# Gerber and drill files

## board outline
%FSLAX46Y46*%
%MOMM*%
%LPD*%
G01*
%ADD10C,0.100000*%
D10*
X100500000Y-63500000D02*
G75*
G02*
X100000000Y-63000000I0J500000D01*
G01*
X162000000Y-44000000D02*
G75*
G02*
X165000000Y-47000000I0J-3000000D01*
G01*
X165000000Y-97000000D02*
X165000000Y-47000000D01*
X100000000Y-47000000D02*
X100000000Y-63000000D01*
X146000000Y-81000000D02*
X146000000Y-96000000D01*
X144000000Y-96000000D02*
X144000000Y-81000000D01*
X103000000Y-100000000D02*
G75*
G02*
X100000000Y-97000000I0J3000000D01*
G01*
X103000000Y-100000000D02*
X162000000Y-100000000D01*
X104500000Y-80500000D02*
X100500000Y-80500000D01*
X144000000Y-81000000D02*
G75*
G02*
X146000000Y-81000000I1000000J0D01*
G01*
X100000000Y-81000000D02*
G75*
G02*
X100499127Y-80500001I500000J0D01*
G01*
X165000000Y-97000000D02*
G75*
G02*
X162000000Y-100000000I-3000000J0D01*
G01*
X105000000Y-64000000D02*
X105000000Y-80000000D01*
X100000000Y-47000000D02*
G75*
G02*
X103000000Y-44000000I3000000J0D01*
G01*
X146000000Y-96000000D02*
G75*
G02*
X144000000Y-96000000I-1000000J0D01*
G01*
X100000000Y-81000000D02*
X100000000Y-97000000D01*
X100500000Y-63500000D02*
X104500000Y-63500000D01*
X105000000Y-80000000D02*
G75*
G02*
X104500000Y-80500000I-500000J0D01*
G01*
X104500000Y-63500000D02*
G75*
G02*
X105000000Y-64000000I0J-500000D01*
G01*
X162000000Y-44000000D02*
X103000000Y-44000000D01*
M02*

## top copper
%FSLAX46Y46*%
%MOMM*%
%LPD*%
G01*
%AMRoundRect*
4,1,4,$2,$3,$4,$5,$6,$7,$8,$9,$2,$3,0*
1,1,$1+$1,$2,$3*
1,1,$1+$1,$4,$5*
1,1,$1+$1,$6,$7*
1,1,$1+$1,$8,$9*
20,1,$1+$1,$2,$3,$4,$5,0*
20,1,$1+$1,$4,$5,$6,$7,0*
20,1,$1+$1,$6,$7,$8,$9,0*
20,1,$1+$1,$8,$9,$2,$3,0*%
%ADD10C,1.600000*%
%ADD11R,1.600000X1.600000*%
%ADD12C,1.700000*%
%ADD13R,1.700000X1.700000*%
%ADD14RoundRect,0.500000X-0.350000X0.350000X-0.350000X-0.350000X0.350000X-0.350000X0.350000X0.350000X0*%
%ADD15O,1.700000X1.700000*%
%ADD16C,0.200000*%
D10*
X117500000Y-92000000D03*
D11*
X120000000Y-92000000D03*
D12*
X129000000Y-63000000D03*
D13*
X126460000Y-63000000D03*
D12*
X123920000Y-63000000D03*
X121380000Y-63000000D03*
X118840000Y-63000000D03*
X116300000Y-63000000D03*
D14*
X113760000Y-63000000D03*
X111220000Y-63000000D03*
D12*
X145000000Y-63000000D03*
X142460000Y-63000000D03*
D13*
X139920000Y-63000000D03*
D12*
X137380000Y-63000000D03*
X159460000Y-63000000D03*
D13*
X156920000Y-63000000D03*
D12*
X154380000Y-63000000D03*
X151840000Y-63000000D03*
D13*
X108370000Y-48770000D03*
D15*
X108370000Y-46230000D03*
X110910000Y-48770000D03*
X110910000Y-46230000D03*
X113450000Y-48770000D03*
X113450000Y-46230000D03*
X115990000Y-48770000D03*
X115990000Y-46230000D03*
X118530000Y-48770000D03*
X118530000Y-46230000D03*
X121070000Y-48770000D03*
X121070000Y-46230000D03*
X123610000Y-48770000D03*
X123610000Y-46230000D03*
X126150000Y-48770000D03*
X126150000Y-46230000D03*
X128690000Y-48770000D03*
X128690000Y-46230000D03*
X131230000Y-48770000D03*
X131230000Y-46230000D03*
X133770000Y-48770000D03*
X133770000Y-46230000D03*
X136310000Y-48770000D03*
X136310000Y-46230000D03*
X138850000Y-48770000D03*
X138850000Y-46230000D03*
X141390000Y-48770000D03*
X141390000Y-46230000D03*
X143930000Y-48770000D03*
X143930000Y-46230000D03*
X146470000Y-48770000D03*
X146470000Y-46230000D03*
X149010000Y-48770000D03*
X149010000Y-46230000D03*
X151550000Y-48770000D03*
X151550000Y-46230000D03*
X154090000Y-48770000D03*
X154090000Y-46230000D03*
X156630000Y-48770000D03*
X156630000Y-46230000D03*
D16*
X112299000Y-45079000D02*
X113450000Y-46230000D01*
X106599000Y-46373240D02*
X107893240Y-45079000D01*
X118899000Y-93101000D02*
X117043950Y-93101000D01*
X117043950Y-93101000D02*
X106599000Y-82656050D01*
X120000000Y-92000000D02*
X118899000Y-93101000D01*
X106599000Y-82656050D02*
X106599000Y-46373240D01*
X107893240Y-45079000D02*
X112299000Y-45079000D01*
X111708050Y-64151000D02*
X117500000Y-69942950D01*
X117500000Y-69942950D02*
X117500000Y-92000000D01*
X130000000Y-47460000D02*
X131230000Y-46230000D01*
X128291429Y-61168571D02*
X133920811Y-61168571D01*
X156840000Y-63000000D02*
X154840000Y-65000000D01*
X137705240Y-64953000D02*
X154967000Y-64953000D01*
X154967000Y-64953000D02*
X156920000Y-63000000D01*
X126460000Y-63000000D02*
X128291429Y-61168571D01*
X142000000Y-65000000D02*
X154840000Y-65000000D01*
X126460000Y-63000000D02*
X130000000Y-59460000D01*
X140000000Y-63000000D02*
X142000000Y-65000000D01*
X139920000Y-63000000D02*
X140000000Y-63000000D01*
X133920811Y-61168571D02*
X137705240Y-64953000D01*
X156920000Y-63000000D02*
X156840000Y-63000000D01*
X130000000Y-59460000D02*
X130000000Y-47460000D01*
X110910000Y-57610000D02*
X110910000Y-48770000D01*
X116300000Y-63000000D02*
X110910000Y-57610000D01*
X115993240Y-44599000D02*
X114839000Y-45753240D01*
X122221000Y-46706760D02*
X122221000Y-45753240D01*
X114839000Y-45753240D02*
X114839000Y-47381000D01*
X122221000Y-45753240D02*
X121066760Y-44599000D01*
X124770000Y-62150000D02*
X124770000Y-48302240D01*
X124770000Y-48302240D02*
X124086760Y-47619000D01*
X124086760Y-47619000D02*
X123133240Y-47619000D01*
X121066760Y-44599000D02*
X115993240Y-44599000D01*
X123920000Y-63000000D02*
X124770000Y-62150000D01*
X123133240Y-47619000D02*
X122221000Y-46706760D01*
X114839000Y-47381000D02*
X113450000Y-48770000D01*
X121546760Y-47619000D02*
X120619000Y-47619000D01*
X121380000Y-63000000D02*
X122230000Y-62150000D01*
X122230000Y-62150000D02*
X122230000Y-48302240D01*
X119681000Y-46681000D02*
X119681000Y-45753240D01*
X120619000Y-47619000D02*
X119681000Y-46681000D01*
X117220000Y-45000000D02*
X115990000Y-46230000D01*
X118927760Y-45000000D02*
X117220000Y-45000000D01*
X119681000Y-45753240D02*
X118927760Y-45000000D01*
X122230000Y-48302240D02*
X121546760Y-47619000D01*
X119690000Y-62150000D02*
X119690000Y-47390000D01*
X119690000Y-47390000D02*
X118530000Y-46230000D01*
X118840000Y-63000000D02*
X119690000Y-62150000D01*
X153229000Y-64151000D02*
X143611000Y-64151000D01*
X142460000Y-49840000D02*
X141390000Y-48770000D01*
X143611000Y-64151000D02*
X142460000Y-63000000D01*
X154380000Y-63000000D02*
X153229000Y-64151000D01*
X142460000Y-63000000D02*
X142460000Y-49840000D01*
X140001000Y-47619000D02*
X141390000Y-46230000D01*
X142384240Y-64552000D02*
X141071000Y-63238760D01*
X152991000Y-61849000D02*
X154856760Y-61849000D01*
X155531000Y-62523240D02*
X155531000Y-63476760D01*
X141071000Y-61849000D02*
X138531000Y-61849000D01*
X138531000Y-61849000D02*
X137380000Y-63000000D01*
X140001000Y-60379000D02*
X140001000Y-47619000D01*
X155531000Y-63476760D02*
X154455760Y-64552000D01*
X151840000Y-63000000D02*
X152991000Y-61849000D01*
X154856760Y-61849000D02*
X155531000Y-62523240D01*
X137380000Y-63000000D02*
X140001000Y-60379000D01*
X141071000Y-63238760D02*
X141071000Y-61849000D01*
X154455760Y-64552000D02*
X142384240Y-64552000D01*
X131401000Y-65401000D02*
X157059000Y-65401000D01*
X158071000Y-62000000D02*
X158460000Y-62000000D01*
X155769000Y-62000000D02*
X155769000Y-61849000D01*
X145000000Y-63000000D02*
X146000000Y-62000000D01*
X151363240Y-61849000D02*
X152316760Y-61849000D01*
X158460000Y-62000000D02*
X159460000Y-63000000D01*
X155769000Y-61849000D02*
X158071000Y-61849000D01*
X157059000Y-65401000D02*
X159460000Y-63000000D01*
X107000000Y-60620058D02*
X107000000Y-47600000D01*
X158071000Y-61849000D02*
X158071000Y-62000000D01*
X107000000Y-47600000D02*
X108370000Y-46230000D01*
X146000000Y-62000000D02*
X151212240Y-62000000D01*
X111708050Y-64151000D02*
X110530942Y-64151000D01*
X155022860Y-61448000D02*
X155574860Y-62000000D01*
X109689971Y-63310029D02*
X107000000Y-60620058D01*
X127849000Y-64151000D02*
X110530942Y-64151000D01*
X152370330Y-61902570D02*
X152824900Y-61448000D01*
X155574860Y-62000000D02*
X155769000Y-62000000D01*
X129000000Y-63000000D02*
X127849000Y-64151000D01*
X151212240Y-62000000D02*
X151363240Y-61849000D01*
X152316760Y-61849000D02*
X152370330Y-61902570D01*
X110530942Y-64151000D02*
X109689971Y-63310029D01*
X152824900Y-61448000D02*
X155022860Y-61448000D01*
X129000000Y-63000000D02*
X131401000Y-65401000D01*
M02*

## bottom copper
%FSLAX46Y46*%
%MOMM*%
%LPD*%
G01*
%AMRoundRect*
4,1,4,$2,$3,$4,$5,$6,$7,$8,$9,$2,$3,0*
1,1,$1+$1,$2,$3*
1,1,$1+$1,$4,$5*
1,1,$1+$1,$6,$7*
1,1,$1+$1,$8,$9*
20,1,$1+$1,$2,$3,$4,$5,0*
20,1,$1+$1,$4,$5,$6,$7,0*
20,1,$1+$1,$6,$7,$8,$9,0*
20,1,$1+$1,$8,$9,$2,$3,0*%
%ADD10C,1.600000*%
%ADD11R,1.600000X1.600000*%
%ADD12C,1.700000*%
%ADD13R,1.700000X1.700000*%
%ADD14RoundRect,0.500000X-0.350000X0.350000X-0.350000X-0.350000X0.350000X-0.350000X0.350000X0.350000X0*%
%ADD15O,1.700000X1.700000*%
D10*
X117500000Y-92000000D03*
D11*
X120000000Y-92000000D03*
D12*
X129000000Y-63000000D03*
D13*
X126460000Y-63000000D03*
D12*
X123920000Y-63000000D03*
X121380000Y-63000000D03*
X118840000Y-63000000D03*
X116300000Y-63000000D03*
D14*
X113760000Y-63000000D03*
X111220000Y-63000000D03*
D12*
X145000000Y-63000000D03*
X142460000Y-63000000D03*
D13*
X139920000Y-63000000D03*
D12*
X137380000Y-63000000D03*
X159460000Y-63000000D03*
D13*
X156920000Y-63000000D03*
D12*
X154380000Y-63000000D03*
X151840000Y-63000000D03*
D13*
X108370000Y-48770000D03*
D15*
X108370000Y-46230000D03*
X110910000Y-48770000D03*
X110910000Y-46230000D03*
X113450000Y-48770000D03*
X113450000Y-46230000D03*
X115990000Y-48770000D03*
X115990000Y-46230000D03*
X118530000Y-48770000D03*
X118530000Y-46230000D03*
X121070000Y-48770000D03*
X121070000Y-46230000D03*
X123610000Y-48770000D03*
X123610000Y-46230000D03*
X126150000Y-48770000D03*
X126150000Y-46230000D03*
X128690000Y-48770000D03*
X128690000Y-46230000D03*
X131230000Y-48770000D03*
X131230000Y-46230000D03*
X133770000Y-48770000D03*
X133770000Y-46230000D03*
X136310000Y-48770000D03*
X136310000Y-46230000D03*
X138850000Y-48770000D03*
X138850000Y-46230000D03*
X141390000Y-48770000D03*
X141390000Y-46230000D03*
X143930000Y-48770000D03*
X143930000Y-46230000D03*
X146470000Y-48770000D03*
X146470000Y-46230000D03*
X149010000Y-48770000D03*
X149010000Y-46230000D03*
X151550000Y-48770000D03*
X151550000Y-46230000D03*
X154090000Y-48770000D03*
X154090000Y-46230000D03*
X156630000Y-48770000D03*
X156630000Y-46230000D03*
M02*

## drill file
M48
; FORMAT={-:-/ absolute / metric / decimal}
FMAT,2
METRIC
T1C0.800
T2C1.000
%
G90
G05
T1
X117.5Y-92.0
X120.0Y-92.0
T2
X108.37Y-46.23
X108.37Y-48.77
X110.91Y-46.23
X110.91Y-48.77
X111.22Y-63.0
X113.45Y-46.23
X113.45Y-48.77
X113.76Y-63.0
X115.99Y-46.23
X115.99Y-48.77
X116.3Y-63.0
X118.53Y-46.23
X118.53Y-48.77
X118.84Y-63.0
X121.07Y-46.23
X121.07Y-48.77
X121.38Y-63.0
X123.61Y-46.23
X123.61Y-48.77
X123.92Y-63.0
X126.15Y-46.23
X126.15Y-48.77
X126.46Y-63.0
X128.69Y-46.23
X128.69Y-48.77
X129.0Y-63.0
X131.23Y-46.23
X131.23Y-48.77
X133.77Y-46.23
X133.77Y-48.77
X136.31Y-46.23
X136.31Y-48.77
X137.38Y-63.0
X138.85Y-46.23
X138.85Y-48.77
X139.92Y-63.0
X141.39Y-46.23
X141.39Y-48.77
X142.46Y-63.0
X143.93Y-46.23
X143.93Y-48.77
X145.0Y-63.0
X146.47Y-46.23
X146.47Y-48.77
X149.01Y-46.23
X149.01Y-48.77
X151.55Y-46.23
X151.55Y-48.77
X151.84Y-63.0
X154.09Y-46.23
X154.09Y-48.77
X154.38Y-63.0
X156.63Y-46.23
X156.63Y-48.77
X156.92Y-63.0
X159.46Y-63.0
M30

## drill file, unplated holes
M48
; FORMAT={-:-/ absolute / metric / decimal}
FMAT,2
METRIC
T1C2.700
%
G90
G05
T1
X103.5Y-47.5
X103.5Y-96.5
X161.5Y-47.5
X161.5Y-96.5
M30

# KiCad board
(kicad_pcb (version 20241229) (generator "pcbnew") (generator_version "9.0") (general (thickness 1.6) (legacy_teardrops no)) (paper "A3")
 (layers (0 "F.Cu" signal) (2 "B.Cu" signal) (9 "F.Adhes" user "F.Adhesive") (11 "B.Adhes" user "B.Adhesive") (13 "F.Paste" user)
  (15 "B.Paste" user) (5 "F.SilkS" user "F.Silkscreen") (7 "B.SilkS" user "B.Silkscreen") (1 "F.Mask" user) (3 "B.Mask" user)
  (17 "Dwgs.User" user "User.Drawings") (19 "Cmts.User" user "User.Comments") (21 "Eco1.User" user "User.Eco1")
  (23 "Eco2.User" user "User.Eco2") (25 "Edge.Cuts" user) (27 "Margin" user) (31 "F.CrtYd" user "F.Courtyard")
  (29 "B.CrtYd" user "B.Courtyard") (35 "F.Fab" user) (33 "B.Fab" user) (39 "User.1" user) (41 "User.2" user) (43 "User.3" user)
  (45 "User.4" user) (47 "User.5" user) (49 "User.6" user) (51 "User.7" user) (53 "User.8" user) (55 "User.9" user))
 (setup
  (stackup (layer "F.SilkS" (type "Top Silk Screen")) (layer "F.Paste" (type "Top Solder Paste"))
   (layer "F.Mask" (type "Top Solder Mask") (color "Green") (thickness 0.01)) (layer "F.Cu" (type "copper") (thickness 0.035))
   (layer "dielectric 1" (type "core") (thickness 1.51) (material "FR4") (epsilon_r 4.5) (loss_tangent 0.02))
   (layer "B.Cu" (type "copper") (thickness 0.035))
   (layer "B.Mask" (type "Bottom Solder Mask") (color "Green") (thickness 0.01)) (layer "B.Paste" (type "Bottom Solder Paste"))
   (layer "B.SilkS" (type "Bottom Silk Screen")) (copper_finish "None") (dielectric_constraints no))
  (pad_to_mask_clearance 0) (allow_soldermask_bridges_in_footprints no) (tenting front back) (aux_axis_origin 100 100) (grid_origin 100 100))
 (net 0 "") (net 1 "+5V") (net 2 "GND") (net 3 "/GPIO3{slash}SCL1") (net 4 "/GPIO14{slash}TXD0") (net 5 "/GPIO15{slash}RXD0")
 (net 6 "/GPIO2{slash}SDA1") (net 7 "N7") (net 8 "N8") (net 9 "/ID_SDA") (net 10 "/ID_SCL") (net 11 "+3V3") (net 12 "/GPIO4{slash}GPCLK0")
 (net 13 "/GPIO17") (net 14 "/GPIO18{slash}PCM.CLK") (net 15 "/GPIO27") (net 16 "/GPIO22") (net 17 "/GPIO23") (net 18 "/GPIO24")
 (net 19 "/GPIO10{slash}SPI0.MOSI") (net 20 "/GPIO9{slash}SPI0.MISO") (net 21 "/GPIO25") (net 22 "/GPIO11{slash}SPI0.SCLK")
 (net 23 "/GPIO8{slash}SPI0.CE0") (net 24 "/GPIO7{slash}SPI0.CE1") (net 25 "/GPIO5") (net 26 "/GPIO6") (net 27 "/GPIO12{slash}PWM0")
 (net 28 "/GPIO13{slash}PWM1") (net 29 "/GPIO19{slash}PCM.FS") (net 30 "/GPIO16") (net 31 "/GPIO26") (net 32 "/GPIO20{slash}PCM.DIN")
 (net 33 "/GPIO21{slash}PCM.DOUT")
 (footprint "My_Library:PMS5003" (layer "F.Cu") (at 121.38 63 -90)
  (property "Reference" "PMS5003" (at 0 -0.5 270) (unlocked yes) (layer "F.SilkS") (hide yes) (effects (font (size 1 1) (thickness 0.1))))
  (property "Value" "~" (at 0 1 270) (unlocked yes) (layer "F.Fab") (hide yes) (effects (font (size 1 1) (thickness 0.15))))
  (pad "1" thru_hole circle (at 0 -7.62 270) (size 1.7 1.7) (drill 1) (layers "*.Cu" "*.Mask") (remove_unused_layers no) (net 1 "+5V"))
  (pad "2" thru_hole rect (at 0 -5.08 270) (size 1.7 1.7) (drill 1) (layers "*.Cu" "*.Mask") (remove_unused_layers no) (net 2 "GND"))
  (pad "3" thru_hole circle (at 0 -2.54 270) (size 1.7 1.7) (drill 1) (layers "*.Cu" "*.Mask") (remove_unused_layers no)
   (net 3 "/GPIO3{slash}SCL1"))
  (pad "4" thru_hole circle (at 0 0 270) (size 1.7 1.7) (drill 1) (layers "*.Cu" "*.Mask") (remove_unused_layers no)
   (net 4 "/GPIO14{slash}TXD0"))
  (pad "5" thru_hole circle (at 0 2.54 270) (size 1.7 1.7) (drill 1) (layers "*.Cu" "*.Mask") (remove_unused_layers no)
   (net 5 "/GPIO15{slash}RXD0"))
  (pad "6" thru_hole circle (at 0 5.08 270) (size 1.7 1.7) (drill 1) (layers "*.Cu" "*.Mask") (remove_unused_layers no)
   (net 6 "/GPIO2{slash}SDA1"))
  (pad "7" thru_hole roundrect (at 0 7.62 270) (size 1.7 1.7) (drill 1) (layers "*.Cu" "*.Mask") (remove_unused_layers no)
   (roundrect_rratio 0.2941176471) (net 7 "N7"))
  (pad "8" thru_hole roundrect (at 0 10.16 270) (size 1.7 1.7) (drill 1) (layers "*.Cu" "*.Mask") (remove_unused_layers no)
   (roundrect_rratio 0.2941176471) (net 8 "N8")))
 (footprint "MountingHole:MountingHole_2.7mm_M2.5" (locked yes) (layer "F.Cu") (at 161.5 47.5)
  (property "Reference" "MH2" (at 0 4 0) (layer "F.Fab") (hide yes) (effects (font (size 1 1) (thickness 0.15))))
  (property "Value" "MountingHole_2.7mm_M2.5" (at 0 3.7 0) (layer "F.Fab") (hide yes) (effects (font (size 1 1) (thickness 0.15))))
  (pad "" np_thru_hole circle (at 0 0) (size 2.7 2.7) (drill 2.7) (layers "*.Cu" "*.Mask")))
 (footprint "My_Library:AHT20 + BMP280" (layer "F.Cu") (at 142.46 63 -90)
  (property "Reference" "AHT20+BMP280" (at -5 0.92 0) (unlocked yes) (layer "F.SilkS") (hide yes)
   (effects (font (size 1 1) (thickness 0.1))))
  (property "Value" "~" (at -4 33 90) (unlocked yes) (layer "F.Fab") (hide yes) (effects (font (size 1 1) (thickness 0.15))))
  (pad "1" thru_hole circle (at 0 -2.54 270) (size 1.7 1.7) (drill 1) (layers "*.Cu" "*.Mask") (remove_unused_layers no) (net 1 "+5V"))
  (pad "2" thru_hole circle (at 0 0 270) (size 1.7 1.7) (drill 1) (layers "*.Cu" "*.Mask") (remove_unused_layers no) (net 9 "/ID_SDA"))
  (pad "3" thru_hole rect (at 0 2.54 270) (size 1.7 1.7) (drill 1) (layers "*.Cu" "*.Mask") (remove_unused_layers no) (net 2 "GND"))
  (pad "4" thru_hole circle (at 0 5.08 270) (size 1.7 1.7) (drill 1) (layers "*.Cu" "*.Mask") (remove_unused_layers no) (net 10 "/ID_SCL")))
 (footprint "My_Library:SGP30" (layer "F.Cu") (at 156.92 63 -90)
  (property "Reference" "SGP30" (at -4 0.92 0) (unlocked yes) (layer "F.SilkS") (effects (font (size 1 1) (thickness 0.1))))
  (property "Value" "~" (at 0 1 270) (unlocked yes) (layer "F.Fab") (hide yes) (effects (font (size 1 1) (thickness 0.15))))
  (pad "1" thru_hole circle (at 0 -2.54 270) (size 1.7 1.7) (drill 1) (layers "*.Cu" "*.Mask") (remove_unused_layers no) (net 1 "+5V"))
  (pad "2" thru_hole rect (at 0 0 270) (size 1.7 1.7) (drill 1) (layers "*.Cu" "*.Mask") (remove_unused_layers no) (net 2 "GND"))
  (pad "3" thru_hole circle (at 0 2.54 270) (size 1.7 1.7) (drill 1) (layers "*.Cu" "*.Mask") (remove_unused_layers no) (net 9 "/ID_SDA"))
  (pad "4" thru_hole circle (at 0 5.08 270) (size 1.7 1.7) (drill 1) (layers "*.Cu" "*.Mask") (remove_unused_layers no) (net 10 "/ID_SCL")))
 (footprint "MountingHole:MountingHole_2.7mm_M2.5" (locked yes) (layer "F.Cu") (at 103.5 96.5)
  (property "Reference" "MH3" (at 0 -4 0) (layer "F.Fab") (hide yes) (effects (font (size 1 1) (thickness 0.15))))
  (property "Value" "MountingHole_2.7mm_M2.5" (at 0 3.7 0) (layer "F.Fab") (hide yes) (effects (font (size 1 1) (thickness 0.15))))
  (pad "" np_thru_hole circle (at 0 0) (size 2.7 2.7) (drill 2.7) (layers "*.Cu" "*.Mask")))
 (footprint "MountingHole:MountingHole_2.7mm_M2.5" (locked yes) (layer "F.Cu") (at 103.5 47.5)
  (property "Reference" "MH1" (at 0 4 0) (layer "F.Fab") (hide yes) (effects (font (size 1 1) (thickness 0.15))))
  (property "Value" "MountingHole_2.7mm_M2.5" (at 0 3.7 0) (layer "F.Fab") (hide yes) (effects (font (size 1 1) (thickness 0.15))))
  (pad "" np_thru_hole circle (at 0 0) (size 2.7 2.7) (drill 2.7) (layers "*.Cu" "*.Mask")))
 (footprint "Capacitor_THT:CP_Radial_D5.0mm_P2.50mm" (layer "F.Cu") (at 117.5 92)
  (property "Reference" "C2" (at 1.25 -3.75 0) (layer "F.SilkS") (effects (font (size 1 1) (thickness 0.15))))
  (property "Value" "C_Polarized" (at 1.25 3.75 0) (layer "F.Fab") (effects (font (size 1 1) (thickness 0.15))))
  (pad "1" thru_hole circle (at 0 0) (size 1.6 1.6) (drill 0.8) (layers "*.Cu" "*.Mask") (remove_unused_layers no) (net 1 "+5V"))
  (pad "2" thru_hole rect (at 2.5 0) (size 1.6 1.6) (drill 0.8) (layers "*.Cu" "*.Mask") (remove_unused_layers no) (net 2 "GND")))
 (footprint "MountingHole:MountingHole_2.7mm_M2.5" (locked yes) (layer "F.Cu") (at 161.5 96.5)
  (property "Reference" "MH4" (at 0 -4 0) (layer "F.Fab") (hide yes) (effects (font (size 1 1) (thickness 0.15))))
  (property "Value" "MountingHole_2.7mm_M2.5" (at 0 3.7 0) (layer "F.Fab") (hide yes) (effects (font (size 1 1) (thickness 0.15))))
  (pad "" np_thru_hole circle (at 0 0) (size 2.7 2.7) (drill 2.7) (layers "*.Cu" "*.Mask")))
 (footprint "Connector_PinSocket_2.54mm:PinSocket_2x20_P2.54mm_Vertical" (layer "B.Cu") (at 108.37 48.77 -90)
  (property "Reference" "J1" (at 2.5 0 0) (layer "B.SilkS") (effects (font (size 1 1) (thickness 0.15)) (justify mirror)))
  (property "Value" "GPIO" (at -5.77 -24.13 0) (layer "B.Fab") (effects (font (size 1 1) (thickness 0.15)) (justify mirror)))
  (pad "1" thru_hole rect (at 0 0 270) (size 1.7 1.7) (drill 1) (layers "*.Cu" "*.Mask") (remove_unused_layers no) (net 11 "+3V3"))
  (pad "2" thru_hole oval (at -2.54 0 270) (size 1.7 1.7) (drill 1) (layers "*.Cu" "*.Mask") (remove_unused_layers no) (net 1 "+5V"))
  (pad "3" thru_hole oval (at 0 -2.54 270) (size 1.7 1.7) (drill 1) (layers "*.Cu" "*.Mask") (remove_unused_layers no)
   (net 6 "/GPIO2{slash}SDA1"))
  (pad "4" thru_hole oval (at -2.54 -2.54 270) (size 1.7 1.7) (drill 1) (layers "*.Cu" "*.Mask") (remove_unused_layers no) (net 1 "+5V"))
  (pad "5" thru_hole oval (at 0 -5.08 270) (size 1.7 1.7) (drill 1) (layers "*.Cu" "*.Mask") (remove_unused_layers no)
   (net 3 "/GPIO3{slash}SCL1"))
  (pad "6" thru_hole oval (at -2.54 -5.08 270) (size 1.7 1.7) (drill 1) (layers "*.Cu" "*.Mask") (remove_unused_layers no) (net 2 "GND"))
  (pad "7" thru_hole oval (at 0 -7.62 270) (size 1.7 1.7) (drill 1) (layers "*.Cu" "*.Mask") (remove_unused_layers no)
   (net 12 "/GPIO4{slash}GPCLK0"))
  (pad "8" thru_hole oval (at -2.54 -7.62 270) (size 1.7 1.7) (drill 1) (layers "*.Cu" "*.Mask") (remove_unused_layers no)
   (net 4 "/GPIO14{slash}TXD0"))
  (pad "9" thru_hole oval (at 0 -10.16 270) (size 1.7 1.7) (drill 1) (layers "*.Cu" "*.Mask") (remove_unused_layers no) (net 2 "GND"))
  (pad "10" thru_hole oval (at -2.54 -10.16 270) (size 1.7 1.7) (drill 1) (layers "*.Cu" "*.Mask") (remove_unused_layers no)
   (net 5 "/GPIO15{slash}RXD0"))
  (pad "11" thru_hole oval (at 0 -12.7 270) (size 1.7 1.7) (drill 1) (layers "*.Cu" "*.Mask") (remove_unused_layers no) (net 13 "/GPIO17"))
  (pad "12" thru_hole oval (at -2.54 -12.7 270) (size 1.7 1.7) (drill 1) (layers "*.Cu" "*.Mask") (remove_unused_layers no)
   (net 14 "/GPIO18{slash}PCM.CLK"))
  (pad "13" thru_hole oval (at 0 -15.24 270) (size 1.7 1.7) (drill 1) (layers "*.Cu" "*.Mask") (remove_unused_layers no) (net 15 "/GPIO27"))
  (pad "14" thru_hole oval (at -2.54 -15.24 270) (size 1.7 1.7) (drill 1) (layers "*.Cu" "*.Mask") (remove_unused_layers no) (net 2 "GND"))
  (pad "15" thru_hole oval (at 0 -17.78 270) (size 1.7 1.7) (drill 1) (layers "*.Cu" "*.Mask") (remove_unused_layers no) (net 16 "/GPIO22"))
  (pad "16" thru_hole oval (at -2.54 -17.78 270) (size 1.7 1.7) (drill 1) (layers "*.Cu" "*.Mask") (remove_unused_layers no)
   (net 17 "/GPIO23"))
  (pad "17" thru_hole oval (at 0 -20.32 270) (size 1.7 1.7) (drill 1) (layers "*.Cu" "*.Mask") (remove_unused_layers no) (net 11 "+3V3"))
  (pad "18" thru_hole oval (at -2.54 -20.32 270) (size 1.7 1.7) (drill 1) (layers "*.Cu" "*.Mask") (remove_unused_layers no)
   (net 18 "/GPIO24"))
  (pad "19" thru_hole oval (at 0 -22.86 270) (size 1.7 1.7) (drill 1) (layers "*.Cu" "*.Mask") (remove_unused_layers no)
   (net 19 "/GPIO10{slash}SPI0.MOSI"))
  (pad "20" thru_hole oval (at -2.54 -22.86 270) (size 1.7 1.7) (drill 1) (layers "*.Cu" "*.Mask") (remove_unused_layers no) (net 2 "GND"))
  (pad "21" thru_hole oval (at 0 -25.4 270) (size 1.7 1.7) (drill 1) (layers "*.Cu" "*.Mask") (remove_unused_layers no)
   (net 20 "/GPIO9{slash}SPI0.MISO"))
  (pad "22" thru_hole oval (at -2.54 -25.4 270) (size 1.7 1.7) (drill 1) (layers "*.Cu" "*.Mask") (remove_unused_layers no)
   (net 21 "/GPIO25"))
  (pad "23" thru_hole oval (at 0 -27.94 270) (size 1.7 1.7) (drill 1) (layers "*.Cu" "*.Mask") (remove_unused_layers no)
   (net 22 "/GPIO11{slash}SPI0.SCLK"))
  (pad "24" thru_hole oval (at -2.54 -27.94 270) (size 1.7 1.7) (drill 1) (layers "*.Cu" "*.Mask") (remove_unused_layers no)
   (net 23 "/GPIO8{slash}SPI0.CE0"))
  (pad "25" thru_hole oval (at 0 -30.48 270) (size 1.7 1.7) (drill 1) (layers "*.Cu" "*.Mask") (remove_unused_layers no) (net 2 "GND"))
  (pad "26" thru_hole oval (at -2.54 -30.48 270) (size 1.7 1.7) (drill 1) (layers "*.Cu" "*.Mask") (remove_unused_layers no)
   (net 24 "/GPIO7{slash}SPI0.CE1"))
  (pad "27" thru_hole oval (at 0 -33.02 270) (size 1.7 1.7) (drill 1) (layers "*.Cu" "*.Mask") (remove_unused_layers no) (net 9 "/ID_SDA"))
  (pad "28" thru_hole oval (at -2.54 -33.02 270) (size 1.7 1.7) (drill 1) (layers "*.Cu" "*.Mask") (remove_unused_layers no)
   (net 10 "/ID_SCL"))
  (pad "29" thru_hole oval (at 0 -35.56 270) (size 1.7 1.7) (drill 1) (layers "*.Cu" "*.Mask") (remove_unused_layers no) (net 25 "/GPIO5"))
  (pad "30" thru_hole oval (at -2.54 -35.56 270) (size 1.7 1.7) (drill 1) (layers "*.Cu" "*.Mask") (remove_unused_layers no) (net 2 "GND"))
  (pad "31" thru_hole oval (at 0 -38.1 270) (size 1.7 1.7) (drill 1) (layers "*.Cu" "*.Mask") (remove_unused_layers no) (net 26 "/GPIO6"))
  (pad "32" thru_hole oval (at -2.54 -38.1 270) (size 1.7 1.7) (drill 1) (layers "*.Cu" "*.Mask") (remove_unused_layers no)
   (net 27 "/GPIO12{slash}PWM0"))
  (pad "33" thru_hole oval (at 0 -40.64 270) (size 1.7 1.7) (drill 1) (layers "*.Cu" "*.Mask") (remove_unused_layers no)
   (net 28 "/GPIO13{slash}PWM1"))
  (pad "34" thru_hole oval (at -2.54 -40.64 270) (size 1.7 1.7) (drill 1) (layers "*.Cu" "*.Mask") (remove_unused_layers no) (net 2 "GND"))
  (pad "35" thru_hole oval (at 0 -43.18 270) (size 1.7 1.7) (drill 1) (layers "*.Cu" "*.Mask") (remove_unused_layers no)
   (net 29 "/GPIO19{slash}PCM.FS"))
  (pad "36" thru_hole oval (at -2.54 -43.18 270) (size 1.7 1.7) (drill 1) (layers "*.Cu" "*.Mask") (remove_unused_layers no)
   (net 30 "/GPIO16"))
  (pad "37" thru_hole oval (at 0 -45.72 270) (size 1.7 1.7) (drill 1) (layers "*.Cu" "*.Mask") (remove_unused_layers no) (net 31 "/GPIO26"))
  (pad "38" thru_hole oval (at -2.54 -45.72 270) (size 1.7 1.7) (drill 1) (layers "*.Cu" "*.Mask") (remove_unused_layers no)
   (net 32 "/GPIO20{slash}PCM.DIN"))
  (pad "39" thru_hole oval (at 0 -48.26 270) (size 1.7 1.7) (drill 1) (layers "*.Cu" "*.Mask") (remove_unused_layers no) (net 2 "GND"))
  (pad "40" thru_hole oval (at -2.54 -48.26 270) (size 1.7 1.7) (drill 1) (layers "*.Cu" "*.Mask") (remove_unused_layers no)
   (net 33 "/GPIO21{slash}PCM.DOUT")))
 (gr_arc (start 100.5 63.5) (mid 100.146447 63.353553) (end 100 63) (stroke (width 0.1) (type solid)) (layer "Edge.Cuts"))
 (gr_arc (start 162 44) (mid 164.12132 44.87868) (end 165 47) (stroke (width 0.1) (type solid)) (layer "Edge.Cuts"))
 (gr_line (start 165 97) (end 165 47) (stroke (width 0.1) (type solid)) (layer "Edge.Cuts"))
 (gr_line (start 100 47) (end 100 63) (stroke (width 0.1) (type solid)) (layer "Edge.Cuts"))
 (gr_line (start 146 81) (end 146 96) (stroke (width 0.1) (type solid)) (layer "Edge.Cuts"))
 (gr_line (start 144 96) (end 144 81) (stroke (width 0.1) (type solid)) (layer "Edge.Cuts"))
 (gr_arc (start 103 100) (mid 100.87868 99.12132) (end 100 97) (stroke (width 0.1) (type solid)) (layer "Edge.Cuts"))
 (gr_line (start 103 100) (end 162 100) (stroke (width 0.1) (type solid)) (layer "Edge.Cuts"))
 (gr_line (start 104.5 80.5) (end 100.5 80.5) (stroke (width 0.1) (type solid)) (layer "Edge.Cuts"))
 (gr_arc (start 144 81) (mid 145 80) (end 146 81) (stroke (width 0.1) (type solid)) (layer "Edge.Cuts"))
 (gr_arc (start 100 81) (mid 100.146138 80.646755) (end 100.499127 80.500001) (stroke (width 0.1) (type solid)) (layer "Edge.Cuts"))
 (gr_arc (start 165 97) (mid 164.12132 99.12132) (end 162 100) (stroke (width 0.1) (type solid)) (layer "Edge.Cuts"))
 (gr_line (start 105 64) (end 105 80) (stroke (width 0.1) (type solid)) (layer "Edge.Cuts"))
 (gr_arc (start 100 47) (mid 100.87868 44.87868) (end 103 44) (stroke (width 0.1) (type solid)) (layer "Edge.Cuts"))
 (gr_arc (start 146 96) (mid 145 97) (end 144 96) (stroke (width 0.1) (type solid)) (layer "Edge.Cuts"))
 (gr_line (start 100 81) (end 100 97) (stroke (width 0.1) (type solid)) (layer "Edge.Cuts"))
 (gr_line (start 100.5 63.5) (end 104.5 63.5) (stroke (width 0.1) (type solid)) (layer "Edge.Cuts"))
 (gr_arc (start 105 80) (mid 104.853553 80.353553) (end 104.5 80.5) (stroke (width 0.1) (type solid)) (layer "Edge.Cuts"))
 (gr_arc (start 104.5 63.5) (mid 104.853553 63.646447) (end 105 64) (stroke (width 0.1) (type solid)) (layer "Edge.Cuts"))
 (gr_line (start 162 44) (end 103 44) (stroke (width 0.1) (type solid)) (layer "Edge.Cuts"))
 (segment (start 130 47.46) (end 131.23 46.23) (width 0.2) (layer "F.Cu") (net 2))
 (segment (start 106.599 82.65605) (end 106.599 46.37324) (width 0.2) (layer "F.Cu") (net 2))
 (segment (start 128.291429 61.168571) (end 133.920811 61.168571) (width 0.2) (layer "F.Cu") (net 2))
 (segment (start 106.599 46.37324) (end 107.89324 45.079) (width 0.2) (layer "F.Cu") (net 2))
 (segment (start 118.899 93.101) (end 117.04395 93.101) (width 0.2) (layer "F.Cu") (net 2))
 (segment (start 156.84 63) (end 154.84 65) (width 0.2) (layer "F.Cu") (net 2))
 (segment (start 137.70524 64.953) (end 154.967 64.953) (width 0.2) (layer "F.Cu") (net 2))
 (segment (start 154.967 64.953) (end 156.92 63) (width 0.2) (layer "F.Cu") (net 2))
 (segment (start 126.46 63) (end 128.291429 61.168571) (width 0.2) (layer "F.Cu") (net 2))
 (segment (start 142 65) (end 154.84 65) (width 0.2) (layer "F.Cu") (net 2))
 (segment (start 126.46 63) (end 130 59.46) (width 0.2) (layer "F.Cu") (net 2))
 (segment (start 117.04395 93.101) (end 106.599 82.65605) (width 0.2) (layer "F.Cu") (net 2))
 (segment (start 140 63) (end 142 65) (width 0.2) (layer "F.Cu") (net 2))
 (segment (start 107.89324 45.079) (end 112.299 45.079) (width 0.2) (layer "F.Cu") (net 2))
 (segment (start 139.92 63) (end 140 63) (width 0.2) (layer "F.Cu") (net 2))
 (segment (start 133.920811 61.168571) (end 137.70524 64.953) (width 0.2) (layer "F.Cu") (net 2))
 (segment (start 156.92 63) (end 156.84 63) (width 0.2) (layer "F.Cu") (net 2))
 (segment (start 120 92) (end 118.899 93.101) (width 0.2) (layer "F.Cu") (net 2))
 (segment (start 112.299 45.079) (end 113.45 46.23) (width 0.2) (layer "F.Cu") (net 2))
 (segment (start 130 59.46) (end 130 47.46) (width 0.2) (layer "F.Cu") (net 2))
 (segment (start 110.91 57.61) (end 110.91 48.77) (width 0.2) (layer "F.Cu") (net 6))
 (segment (start 116.3 63) (end 110.91 57.61) (width 0.2) (layer "F.Cu") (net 6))
 (segment (start 115.99324 44.599) (end 114.839 45.75324) (width 0.2) (layer "F.Cu") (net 3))
 (segment (start 122.221 46.70676) (end 122.221 45.75324) (width 0.2) (layer "F.Cu") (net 3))
 (segment (start 114.839 45.75324) (end 114.839 47.381) (width 0.2) (layer "F.Cu") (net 3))
 (segment (start 122.221 45.75324) (end 121.06676 44.599) (width 0.2) (layer "F.Cu") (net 3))
 (segment (start 124.77 62.15) (end 124.77 48.30224) (width 0.2) (layer "F.Cu") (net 3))
 (segment (start 124.77 48.30224) (end 124.08676 47.619) (width 0.2) (layer "F.Cu") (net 3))
 (segment (start 124.08676 47.619) (end 123.13324 47.619) (width 0.2) (layer "F.Cu") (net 3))
 (segment (start 121.06676 44.599) (end 115.99324 44.599) (width 0.2) (layer "F.Cu") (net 3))
 (segment (start 123.92 63) (end 124.77 62.15) (width 0.2) (layer "F.Cu") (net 3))
 (segment (start 123.13324 47.619) (end 122.221 46.70676) (width 0.2) (layer "F.Cu") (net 3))
 (segment (start 114.839 47.381) (end 113.45 48.77) (width 0.2) (layer "F.Cu") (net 3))
 (segment (start 121.54676 47.619) (end 120.619 47.619) (width 0.2) (layer "F.Cu") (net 4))
 (segment (start 121.38 63) (end 122.23 62.15) (width 0.2) (layer "F.Cu") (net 4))
 (segment (start 122.23 62.15) (end 122.23 48.30224) (width 0.2) (layer "F.Cu") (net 4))
 (segment (start 119.681 46.681) (end 119.681 45.75324) (width 0.2) (layer "F.Cu") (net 4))
 (segment (start 120.619 47.619) (end 119.681 46.681) (width 0.2) (layer "F.Cu") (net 4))
 (segment (start 117.22 45) (end 115.99 46.23) (width 0.2) (layer "F.Cu") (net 4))
 (segment (start 118.92776 45) (end 117.22 45) (width 0.2) (layer "F.Cu") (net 4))
 (segment (start 119.681 45.75324) (end 118.92776 45) (width 0.2) (layer "F.Cu") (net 4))
 (segment (start 122.23 48.30224) (end 121.54676 47.619) (width 0.2) (layer "F.Cu") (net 4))
 (segment (start 119.69 62.15) (end 119.69 47.39) (width 0.2) (layer "F.Cu") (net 5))
 (segment (start 119.69 47.39) (end 118.53 46.23) (width 0.2) (layer "F.Cu") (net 5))
 (segment (start 118.84 63) (end 119.69 62.15) (width 0.2) (layer "F.Cu") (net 5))
 (segment (start 153.229 64.151) (end 143.611 64.151) (width 0.2) (layer "F.Cu") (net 9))
 (segment (start 142.46 49.84) (end 141.39 48.77) (width 0.2) (layer "F.Cu") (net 9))
 (segment (start 143.611 64.151) (end 142.46 63) (width 0.2) (layer "F.Cu") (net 9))
 (segment (start 154.38 63) (end 153.229 64.151) (width 0.2) (layer "F.Cu") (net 9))
 (segment (start 142.46 63) (end 142.46 49.84) (width 0.2) (layer "F.Cu") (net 9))
 (segment (start 140.001 47.619) (end 141.39 46.23) (width 0.2) (layer "F.Cu") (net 10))
 (segment (start 142.38424 64.552) (end 141.071 63.23876) (width 0.2) (layer "F.Cu") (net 10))
 (segment (start 152.991 61.849) (end 154.85676 61.849) (width 0.2) (layer "F.Cu") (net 10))
 (segment (start 155.531 62.52324) (end 155.531 63.47676) (width 0.2) (layer "F.Cu") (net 10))
 (segment (start 141.071 61.849) (end 138.531 61.849) (width 0.2) (layer "F.Cu") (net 10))
 (segment (start 138.531 61.849) (end 137.38 63) (width 0.2) (layer "F.Cu") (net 10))
 (segment (start 140.001 60.379) (end 140.001 47.619) (width 0.2) (layer "F.Cu") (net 10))
 (segment (start 155.531 63.47676) (end 154.45576 64.552) (width 0.2) (layer "F.Cu") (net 10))
 (segment (start 151.84 63) (end 152.991 61.849) (width 0.2) (layer "F.Cu") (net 10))
 (segment (start 154.85676 61.849) (end 155.531 62.52324) (width 0.2) (layer "F.Cu") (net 10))
 (segment (start 137.38 63) (end 140.001 60.379) (width 0.2) (layer "F.Cu") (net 10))
 (segment (start 141.071 63.23876) (end 141.071 61.849) (width 0.2) (layer "F.Cu") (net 10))
 (segment (start 154.45576 64.552) (end 142.38424 64.552) (width 0.2) (layer "F.Cu") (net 10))
 (segment (start 131.401 65.401) (end 157.059 65.401) (width 0.2) (layer "F.Cu") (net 1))
 (segment (start 158.071 62) (end 158.46 62) (width 0.2) (layer "F.Cu") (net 1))
 (segment (start 117.5 69.94295) (end 117.5 92) (width 0.2) (layer "F.Cu") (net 1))
 (segment (start 155.769 62) (end 155.769 61.849) (width 0.2) (layer "F.Cu") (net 1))
 (segment (start 145 63) (end 146 62) (width 0.2) (layer "F.Cu") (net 1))
 (segment (start 151.36324 61.849) (end 152.31676 61.849) (width 0.2) (layer "F.Cu") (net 1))
 (segment (start 158.46 62) (end 159.46 63) (width 0.2) (layer "F.Cu") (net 1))
 (segment (start 155.769 61.849) (end 158.071 61.849) (width 0.2) (layer "F.Cu") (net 1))
 (segment (start 157.059 65.401) (end 159.46 63) (width 0.2) (layer "F.Cu") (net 1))
 (segment (start 107 60.620058) (end 107 47.6) (width 0.2) (layer "F.Cu") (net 1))
 (segment (start 158.071 61.849) (end 158.071 62) (width 0.2) (layer "F.Cu") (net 1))
 (segment (start 107 47.6) (end 108.37 46.23) (width 0.2) (layer "F.Cu") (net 1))
 (segment (start 146 62) (end 151.21224 62) (width 0.2) (layer "F.Cu") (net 1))
 (segment (start 111.70805 64.151) (end 110.530942 64.151) (width 0.2) (layer "F.Cu") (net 1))
 (segment (start 155.02286 61.448) (end 155.57486 62) (width 0.2) (layer "F.Cu") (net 1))
 (segment (start 109.689971 63.310029) (end 107 60.620058) (width 0.2) (layer "F.Cu") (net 1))
 (segment (start 127.849 64.151) (end 110.530942 64.151) (width 0.2) (layer "F.Cu") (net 1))
 (segment (start 152.37033 61.90257) (end 152.8249 61.448) (width 0.2) (layer "F.Cu") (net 1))
 (segment (start 155.57486 62) (end 155.769 62) (width 0.2) (layer "F.Cu") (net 1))
 (segment (start 129 63) (end 127.849 64.151) (width 0.2) (layer "F.Cu") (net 1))
 (segment (start 151.21224 62) (end 151.36324 61.849) (width 0.2) (layer "F.Cu") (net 1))
 (segment (start 152.31676 61.849) (end 152.37033 61.90257) (width 0.2) (layer "F.Cu") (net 1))
 (segment (start 110.530942 64.151) (end 109.689971 63.310029) (width 0.2) (layer "F.Cu") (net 1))
 (segment (start 152.8249 61.448) (end 155.02286 61.448) (width 0.2) (layer "F.Cu") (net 1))
 (segment (start 129 63) (end 131.401 65.401) (width 0.2) (layer "F.Cu") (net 1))
 (segment (start 111.70805 64.151) (end 117.5 69.94295) (width 0.2) (layer "F.Cu") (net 1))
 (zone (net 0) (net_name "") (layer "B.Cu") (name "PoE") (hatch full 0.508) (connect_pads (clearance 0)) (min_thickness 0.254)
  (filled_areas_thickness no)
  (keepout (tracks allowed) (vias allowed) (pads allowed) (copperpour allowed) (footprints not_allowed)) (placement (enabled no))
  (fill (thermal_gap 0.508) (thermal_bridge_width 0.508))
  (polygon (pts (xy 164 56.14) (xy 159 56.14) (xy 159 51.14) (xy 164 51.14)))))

